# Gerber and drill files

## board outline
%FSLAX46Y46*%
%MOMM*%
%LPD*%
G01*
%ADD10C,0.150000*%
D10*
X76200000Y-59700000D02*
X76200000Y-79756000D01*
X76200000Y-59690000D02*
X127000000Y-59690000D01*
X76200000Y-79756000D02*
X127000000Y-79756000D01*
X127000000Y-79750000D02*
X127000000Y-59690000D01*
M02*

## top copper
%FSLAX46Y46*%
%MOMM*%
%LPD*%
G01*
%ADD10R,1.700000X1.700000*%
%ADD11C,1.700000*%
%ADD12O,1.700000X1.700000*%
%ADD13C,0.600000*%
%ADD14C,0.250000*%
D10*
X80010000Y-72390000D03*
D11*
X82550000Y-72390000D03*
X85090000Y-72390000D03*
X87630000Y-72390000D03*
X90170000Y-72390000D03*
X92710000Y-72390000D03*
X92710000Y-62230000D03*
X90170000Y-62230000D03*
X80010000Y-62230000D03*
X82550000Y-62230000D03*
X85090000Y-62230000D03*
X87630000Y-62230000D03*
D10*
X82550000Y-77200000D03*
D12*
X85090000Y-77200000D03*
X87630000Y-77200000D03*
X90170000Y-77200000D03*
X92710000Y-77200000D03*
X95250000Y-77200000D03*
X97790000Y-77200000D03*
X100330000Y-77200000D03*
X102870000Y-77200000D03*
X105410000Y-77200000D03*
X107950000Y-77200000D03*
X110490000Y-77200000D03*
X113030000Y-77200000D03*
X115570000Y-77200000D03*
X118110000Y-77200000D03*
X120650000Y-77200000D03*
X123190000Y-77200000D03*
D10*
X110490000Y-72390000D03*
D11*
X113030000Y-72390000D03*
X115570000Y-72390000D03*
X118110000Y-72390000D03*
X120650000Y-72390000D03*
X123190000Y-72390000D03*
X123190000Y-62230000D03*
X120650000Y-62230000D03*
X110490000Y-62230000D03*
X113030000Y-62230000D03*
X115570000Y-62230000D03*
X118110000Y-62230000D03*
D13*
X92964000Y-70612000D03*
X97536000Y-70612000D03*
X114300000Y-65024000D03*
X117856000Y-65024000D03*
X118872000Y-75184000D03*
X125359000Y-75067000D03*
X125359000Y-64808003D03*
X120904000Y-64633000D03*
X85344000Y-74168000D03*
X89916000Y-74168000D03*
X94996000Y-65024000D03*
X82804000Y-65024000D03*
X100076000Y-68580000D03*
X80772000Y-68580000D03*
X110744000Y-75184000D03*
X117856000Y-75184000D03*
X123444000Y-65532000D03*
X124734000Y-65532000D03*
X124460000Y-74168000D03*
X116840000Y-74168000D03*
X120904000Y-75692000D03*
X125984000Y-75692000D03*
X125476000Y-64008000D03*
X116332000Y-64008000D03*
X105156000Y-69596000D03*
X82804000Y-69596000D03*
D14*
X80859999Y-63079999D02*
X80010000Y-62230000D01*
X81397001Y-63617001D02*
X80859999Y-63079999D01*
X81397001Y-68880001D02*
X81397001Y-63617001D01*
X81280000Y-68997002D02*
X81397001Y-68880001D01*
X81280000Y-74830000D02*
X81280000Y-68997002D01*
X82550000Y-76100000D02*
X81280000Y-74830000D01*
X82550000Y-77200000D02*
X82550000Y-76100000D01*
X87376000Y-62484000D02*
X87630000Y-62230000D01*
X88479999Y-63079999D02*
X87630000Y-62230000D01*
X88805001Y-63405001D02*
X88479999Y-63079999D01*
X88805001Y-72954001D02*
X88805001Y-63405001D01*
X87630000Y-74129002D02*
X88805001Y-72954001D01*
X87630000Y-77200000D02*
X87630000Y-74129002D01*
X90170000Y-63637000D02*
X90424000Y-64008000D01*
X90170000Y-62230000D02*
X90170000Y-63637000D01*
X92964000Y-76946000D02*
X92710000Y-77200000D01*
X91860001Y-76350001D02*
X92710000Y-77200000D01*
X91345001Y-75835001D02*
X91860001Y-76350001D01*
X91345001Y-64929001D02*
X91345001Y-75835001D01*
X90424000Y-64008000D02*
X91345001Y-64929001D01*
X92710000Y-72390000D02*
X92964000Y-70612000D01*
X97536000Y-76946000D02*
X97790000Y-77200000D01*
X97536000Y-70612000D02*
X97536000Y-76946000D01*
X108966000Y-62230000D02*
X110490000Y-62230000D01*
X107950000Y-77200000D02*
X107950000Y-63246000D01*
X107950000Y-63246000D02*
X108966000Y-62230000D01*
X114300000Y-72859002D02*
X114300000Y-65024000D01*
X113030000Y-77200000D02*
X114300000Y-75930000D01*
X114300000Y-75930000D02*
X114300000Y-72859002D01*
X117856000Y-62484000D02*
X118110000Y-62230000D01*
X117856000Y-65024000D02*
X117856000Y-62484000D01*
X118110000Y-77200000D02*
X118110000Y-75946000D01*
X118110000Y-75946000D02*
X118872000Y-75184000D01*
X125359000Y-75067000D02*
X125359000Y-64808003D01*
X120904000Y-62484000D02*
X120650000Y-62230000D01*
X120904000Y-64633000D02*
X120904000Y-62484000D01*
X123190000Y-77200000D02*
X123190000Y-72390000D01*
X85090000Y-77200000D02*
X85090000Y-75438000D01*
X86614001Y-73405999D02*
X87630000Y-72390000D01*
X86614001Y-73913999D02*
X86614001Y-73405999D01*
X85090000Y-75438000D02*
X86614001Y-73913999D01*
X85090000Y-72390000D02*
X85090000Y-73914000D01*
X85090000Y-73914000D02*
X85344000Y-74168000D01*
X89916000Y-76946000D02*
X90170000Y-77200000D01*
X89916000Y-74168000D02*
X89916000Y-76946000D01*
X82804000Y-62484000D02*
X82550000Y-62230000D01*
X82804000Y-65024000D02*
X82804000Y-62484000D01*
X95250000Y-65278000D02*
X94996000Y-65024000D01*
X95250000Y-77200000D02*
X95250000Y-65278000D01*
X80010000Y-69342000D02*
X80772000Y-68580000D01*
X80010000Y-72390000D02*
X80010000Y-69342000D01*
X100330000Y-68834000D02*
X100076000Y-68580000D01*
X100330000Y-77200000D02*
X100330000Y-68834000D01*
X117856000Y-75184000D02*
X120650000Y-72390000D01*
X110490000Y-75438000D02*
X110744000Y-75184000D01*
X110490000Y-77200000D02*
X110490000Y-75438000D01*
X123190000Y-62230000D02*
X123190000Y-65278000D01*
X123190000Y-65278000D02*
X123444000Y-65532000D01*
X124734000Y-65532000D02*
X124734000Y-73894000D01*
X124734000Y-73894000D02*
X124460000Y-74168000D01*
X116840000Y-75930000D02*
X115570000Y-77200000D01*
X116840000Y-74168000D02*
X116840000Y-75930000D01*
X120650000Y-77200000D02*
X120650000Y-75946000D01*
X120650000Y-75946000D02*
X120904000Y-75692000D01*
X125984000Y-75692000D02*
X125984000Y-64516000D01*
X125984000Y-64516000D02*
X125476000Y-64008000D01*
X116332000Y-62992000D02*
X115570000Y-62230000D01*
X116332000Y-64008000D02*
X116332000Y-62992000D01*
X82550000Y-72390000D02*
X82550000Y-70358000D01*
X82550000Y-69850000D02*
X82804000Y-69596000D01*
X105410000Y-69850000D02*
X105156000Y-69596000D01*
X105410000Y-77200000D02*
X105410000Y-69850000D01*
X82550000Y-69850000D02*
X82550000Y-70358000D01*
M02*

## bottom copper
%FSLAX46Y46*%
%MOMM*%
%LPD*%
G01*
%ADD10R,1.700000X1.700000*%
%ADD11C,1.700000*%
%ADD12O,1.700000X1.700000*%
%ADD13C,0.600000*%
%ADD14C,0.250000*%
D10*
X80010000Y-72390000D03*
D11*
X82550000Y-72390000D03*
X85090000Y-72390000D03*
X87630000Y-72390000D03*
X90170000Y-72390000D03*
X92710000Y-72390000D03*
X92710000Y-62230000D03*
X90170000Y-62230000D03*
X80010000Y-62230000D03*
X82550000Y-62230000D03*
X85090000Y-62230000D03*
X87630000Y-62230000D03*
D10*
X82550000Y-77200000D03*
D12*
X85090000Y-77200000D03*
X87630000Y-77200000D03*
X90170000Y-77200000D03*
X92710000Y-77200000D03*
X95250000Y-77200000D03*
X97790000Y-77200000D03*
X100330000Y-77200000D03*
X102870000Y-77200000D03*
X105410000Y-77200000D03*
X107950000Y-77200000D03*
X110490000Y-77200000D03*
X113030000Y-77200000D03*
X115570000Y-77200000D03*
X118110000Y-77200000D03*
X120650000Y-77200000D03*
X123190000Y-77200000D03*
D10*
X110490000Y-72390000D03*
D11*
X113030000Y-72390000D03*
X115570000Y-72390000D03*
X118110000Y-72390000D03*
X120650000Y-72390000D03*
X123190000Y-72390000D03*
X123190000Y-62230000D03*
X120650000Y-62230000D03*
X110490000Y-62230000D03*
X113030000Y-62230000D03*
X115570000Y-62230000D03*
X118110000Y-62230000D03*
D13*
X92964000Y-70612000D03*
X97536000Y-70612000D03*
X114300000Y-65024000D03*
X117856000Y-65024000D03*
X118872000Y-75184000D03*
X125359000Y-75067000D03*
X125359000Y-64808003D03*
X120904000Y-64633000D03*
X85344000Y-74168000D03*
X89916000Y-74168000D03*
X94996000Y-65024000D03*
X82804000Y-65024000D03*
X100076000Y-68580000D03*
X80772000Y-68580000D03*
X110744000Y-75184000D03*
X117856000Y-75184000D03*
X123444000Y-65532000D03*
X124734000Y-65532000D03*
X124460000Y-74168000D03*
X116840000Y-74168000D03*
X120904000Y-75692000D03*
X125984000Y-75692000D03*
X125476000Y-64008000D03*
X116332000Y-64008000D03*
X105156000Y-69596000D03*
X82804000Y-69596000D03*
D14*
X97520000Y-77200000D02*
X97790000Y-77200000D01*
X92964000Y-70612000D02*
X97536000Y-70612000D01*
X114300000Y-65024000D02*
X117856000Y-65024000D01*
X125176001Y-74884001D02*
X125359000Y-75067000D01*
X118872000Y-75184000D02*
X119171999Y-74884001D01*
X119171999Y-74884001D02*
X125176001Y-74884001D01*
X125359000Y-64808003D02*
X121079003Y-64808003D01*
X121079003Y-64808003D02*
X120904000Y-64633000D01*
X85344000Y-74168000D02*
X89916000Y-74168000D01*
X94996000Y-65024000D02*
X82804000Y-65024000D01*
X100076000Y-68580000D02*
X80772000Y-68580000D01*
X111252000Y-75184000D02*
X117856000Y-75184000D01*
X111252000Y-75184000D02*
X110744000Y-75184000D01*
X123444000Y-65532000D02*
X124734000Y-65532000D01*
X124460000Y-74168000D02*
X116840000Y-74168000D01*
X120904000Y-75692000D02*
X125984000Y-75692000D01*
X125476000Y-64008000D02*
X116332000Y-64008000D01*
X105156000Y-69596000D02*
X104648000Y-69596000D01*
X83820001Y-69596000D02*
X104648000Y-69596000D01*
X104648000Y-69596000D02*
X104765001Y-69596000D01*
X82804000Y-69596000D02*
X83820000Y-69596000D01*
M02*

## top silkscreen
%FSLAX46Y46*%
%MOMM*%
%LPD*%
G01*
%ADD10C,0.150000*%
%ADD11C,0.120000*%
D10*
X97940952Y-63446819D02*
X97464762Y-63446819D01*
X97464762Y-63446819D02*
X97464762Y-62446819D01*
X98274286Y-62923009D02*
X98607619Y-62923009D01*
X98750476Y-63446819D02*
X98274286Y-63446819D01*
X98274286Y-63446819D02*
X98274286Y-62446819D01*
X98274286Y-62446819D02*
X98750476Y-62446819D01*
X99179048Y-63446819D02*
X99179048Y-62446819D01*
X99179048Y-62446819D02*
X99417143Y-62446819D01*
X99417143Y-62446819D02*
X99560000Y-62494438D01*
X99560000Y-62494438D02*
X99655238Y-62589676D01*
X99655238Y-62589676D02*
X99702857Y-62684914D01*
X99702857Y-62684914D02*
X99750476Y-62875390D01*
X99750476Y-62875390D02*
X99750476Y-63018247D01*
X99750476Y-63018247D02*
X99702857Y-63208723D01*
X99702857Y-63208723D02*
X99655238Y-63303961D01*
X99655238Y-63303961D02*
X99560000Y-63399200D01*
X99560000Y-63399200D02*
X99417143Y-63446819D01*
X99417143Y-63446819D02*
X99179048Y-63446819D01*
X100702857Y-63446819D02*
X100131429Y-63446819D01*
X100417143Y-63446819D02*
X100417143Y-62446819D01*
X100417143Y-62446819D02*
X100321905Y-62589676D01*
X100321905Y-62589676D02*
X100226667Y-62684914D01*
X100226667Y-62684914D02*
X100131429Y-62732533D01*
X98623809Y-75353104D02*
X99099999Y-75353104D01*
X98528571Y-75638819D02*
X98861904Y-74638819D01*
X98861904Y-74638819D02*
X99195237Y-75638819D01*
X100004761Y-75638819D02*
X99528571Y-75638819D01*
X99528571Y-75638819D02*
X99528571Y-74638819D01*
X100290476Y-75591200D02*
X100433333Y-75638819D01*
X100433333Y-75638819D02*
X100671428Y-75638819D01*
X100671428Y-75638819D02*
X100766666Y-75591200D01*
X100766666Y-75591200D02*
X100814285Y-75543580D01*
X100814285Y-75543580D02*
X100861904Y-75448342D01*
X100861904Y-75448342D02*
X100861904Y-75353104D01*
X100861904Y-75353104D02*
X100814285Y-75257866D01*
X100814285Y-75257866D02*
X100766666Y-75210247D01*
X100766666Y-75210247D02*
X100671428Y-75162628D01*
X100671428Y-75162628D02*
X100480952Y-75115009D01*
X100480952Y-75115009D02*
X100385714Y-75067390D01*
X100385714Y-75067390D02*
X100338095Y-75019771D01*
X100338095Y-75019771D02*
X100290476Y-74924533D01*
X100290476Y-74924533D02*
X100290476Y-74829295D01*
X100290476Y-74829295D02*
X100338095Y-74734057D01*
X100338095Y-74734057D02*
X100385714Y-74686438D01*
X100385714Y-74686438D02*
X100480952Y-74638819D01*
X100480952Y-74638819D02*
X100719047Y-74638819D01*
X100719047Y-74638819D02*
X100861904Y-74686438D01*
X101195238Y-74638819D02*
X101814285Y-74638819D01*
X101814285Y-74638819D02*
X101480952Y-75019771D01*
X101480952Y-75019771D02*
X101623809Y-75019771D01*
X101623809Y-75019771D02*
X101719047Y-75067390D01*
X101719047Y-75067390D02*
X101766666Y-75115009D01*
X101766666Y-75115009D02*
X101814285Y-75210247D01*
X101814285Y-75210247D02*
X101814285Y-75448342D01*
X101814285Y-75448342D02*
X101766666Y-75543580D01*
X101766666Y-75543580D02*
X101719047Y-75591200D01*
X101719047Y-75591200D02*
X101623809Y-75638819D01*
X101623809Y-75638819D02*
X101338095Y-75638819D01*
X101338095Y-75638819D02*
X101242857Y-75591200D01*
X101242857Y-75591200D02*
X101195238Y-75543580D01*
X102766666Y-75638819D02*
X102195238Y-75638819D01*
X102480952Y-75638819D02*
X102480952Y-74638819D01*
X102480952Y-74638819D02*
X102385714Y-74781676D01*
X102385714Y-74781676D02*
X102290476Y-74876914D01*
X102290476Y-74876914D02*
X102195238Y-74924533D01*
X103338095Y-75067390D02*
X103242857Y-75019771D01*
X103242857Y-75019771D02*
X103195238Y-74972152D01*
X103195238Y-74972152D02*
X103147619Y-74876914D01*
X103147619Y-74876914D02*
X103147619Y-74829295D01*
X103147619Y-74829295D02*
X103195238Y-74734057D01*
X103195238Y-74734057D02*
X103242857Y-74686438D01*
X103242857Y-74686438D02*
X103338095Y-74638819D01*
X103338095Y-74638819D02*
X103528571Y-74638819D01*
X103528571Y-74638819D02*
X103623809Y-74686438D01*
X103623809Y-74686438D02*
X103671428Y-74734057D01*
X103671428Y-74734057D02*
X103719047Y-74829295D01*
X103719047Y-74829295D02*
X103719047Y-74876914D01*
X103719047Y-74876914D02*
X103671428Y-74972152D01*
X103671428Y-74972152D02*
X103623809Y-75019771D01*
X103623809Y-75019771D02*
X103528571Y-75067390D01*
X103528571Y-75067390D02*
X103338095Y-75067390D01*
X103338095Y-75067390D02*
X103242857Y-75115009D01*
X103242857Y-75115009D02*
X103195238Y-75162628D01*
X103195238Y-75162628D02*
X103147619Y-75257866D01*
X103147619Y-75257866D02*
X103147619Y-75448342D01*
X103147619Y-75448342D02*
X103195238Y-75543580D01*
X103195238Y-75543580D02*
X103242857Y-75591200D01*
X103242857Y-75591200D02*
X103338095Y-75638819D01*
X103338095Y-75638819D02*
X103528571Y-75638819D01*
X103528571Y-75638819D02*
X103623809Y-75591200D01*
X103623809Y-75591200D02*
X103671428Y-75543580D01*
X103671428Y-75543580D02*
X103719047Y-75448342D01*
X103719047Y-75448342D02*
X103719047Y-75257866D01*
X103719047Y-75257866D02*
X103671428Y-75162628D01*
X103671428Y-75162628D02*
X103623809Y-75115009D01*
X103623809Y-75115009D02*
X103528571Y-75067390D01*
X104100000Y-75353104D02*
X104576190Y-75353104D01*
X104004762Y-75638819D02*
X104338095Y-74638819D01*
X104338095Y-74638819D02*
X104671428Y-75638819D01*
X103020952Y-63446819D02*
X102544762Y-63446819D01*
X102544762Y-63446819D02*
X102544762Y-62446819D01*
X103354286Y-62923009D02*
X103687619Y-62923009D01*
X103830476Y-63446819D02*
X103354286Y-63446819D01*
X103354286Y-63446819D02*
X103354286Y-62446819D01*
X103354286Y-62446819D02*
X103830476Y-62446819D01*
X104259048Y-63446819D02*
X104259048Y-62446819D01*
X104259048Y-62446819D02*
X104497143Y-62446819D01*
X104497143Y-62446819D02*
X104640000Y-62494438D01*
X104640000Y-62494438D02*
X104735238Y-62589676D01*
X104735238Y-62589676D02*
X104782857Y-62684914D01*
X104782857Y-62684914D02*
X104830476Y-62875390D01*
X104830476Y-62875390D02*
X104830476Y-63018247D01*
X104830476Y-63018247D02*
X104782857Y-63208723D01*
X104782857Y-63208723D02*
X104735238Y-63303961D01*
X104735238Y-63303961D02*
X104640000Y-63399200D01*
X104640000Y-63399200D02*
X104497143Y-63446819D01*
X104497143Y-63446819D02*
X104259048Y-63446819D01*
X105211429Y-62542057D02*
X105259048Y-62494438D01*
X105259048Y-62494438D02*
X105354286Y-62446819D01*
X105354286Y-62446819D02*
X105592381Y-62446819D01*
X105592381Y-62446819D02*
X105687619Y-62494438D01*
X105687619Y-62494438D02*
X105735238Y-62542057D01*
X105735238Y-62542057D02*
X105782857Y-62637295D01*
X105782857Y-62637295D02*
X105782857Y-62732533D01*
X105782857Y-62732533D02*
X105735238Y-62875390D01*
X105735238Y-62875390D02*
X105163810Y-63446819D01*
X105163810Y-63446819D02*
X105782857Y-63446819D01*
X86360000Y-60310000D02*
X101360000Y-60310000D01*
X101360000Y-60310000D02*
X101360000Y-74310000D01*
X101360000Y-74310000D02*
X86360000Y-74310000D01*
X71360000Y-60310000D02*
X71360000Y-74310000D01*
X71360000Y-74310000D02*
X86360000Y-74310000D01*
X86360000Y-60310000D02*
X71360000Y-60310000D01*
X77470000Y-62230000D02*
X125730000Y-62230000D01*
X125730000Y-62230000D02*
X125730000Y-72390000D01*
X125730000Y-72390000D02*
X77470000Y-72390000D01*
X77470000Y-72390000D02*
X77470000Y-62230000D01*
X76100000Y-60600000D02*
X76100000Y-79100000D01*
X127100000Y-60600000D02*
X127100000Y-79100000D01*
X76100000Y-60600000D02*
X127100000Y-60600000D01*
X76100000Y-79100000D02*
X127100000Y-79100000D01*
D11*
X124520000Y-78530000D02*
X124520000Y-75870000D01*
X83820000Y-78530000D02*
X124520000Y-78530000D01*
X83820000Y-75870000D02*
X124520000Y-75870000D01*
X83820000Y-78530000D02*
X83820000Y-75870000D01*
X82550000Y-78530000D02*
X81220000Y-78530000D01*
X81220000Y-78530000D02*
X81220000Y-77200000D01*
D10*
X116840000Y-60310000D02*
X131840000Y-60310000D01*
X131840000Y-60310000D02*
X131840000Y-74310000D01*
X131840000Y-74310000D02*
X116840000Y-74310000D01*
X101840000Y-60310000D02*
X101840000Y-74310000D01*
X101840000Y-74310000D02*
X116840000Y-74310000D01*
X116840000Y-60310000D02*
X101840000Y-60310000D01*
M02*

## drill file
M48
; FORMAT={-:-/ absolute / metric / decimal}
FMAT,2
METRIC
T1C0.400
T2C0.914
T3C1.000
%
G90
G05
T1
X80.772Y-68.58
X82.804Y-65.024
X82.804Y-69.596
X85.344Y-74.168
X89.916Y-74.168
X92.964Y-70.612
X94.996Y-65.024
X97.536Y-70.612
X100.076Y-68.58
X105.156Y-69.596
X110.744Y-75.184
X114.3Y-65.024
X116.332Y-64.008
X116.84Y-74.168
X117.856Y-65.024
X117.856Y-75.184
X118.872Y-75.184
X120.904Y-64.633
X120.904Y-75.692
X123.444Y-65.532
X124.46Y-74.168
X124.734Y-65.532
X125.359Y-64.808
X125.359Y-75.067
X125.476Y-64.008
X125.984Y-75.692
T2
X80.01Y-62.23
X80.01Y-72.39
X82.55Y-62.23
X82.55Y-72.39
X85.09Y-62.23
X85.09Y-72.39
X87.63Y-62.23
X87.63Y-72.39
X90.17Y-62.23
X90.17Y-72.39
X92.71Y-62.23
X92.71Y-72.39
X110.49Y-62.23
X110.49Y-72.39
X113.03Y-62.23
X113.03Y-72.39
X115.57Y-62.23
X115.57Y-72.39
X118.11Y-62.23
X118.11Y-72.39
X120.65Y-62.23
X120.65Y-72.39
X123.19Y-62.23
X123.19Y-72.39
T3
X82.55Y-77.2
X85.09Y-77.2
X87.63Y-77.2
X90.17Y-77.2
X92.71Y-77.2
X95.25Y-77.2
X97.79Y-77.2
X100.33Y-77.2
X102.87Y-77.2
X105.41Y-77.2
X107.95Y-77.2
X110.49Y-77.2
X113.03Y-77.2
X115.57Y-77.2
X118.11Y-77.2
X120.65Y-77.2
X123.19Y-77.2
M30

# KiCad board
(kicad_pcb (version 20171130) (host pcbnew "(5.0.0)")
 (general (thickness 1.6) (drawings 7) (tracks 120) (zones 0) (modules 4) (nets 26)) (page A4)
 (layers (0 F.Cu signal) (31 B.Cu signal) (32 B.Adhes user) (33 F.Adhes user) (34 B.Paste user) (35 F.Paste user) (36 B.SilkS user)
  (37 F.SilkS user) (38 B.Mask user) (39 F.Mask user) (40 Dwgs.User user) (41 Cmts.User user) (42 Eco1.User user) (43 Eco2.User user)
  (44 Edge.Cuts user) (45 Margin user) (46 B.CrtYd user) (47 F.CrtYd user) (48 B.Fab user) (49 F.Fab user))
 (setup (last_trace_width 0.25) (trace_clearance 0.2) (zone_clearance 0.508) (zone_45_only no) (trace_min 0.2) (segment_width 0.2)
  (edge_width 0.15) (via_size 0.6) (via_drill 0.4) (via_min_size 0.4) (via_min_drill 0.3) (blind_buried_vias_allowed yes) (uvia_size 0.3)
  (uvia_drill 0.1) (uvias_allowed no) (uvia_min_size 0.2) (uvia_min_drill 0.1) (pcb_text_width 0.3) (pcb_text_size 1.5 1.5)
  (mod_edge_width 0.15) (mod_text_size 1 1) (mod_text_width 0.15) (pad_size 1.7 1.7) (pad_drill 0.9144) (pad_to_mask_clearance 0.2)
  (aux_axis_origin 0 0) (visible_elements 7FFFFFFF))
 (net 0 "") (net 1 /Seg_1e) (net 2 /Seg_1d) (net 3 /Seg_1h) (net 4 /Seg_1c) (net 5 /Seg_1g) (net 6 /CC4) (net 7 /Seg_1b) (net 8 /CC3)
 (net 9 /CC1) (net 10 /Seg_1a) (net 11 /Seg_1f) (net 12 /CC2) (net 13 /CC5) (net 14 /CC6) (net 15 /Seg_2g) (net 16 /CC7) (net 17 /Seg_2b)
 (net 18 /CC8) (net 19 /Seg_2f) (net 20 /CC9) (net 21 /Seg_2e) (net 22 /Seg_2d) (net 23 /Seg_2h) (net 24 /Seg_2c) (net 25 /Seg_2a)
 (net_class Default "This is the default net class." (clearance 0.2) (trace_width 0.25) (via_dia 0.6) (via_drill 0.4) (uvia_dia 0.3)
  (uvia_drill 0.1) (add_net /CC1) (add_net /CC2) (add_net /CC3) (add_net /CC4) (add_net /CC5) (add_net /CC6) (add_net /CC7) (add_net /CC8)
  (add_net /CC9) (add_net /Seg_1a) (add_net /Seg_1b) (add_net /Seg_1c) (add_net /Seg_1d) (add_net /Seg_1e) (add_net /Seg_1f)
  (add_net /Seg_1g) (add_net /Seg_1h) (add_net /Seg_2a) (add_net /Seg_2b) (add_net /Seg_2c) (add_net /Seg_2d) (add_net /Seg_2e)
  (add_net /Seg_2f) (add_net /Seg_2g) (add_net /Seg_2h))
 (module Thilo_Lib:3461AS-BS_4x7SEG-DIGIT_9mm (layer F.Cu) (at 86.36 67.31)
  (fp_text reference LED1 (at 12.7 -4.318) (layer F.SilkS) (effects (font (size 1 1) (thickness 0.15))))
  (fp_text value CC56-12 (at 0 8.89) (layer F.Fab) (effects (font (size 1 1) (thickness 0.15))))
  (fp_line (start 0 -7) (end 15 -7) (layer F.SilkS) (width 0.15))
  (fp_line (start 15 -7) (end 15 7) (layer F.SilkS) (width 0.15))
  (fp_line (start 15 7) (end 0 7) (layer F.SilkS) (width 0.15))
  (fp_line (start -15 -7) (end -15 7) (layer F.SilkS) (width 0.15))
  (fp_line (start -15 7) (end 0 7) (layer F.SilkS) (width 0.15))
  (fp_line (start 0 -7) (end -15 -7) (layer F.SilkS) (width 0.15))
  (pad 1 thru_hole rect (at -6.35 5.08) (size 1.7 1.7) (drill 0.9144) (layers *.Cu *.Mask) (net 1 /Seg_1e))
  (pad 2 thru_hole circle (at -3.81 5.08) (size 1.7 1.7) (drill 0.9144) (layers *.Cu *.Mask) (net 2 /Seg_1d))
  (pad 3 thru_hole circle (at -1.27 5.08) (size 1.7 1.7) (drill 0.9144) (layers *.Cu *.Mask) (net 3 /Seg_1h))
  (pad 4 thru_hole circle (at 1.27 5.08) (size 1.7 1.7) (drill 0.9144) (layers *.Cu *.Mask) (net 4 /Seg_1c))
  (pad 5 thru_hole circle (at 3.81 5.08) (size 1.7 1.7) (drill 0.9144) (layers *.Cu *.Mask) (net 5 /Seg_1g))
  (pad 6 thru_hole circle (at 6.35 5.08) (size 1.7 1.7) (drill 0.9144) (layers *.Cu *.Mask) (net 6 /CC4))
  (pad 7 thru_hole circle (at 6.35 -5.08) (size 1.7 1.7) (drill 0.9144) (layers *.Cu *.Mask) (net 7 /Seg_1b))
  (pad 8 thru_hole circle (at 3.81 -5.08) (size 1.7 1.7) (drill 0.9144) (layers *.Cu *.Mask) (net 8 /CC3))
  (pad 12 thru_hole circle (at -6.35 -5.08) (size 1.7 1.7) (drill 0.9144) (layers *.Cu *.Mask) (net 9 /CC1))
  (pad 11 thru_hole circle (at -3.81 -5.08) (size 1.7 1.7) (drill 0.9144) (layers *.Cu *.Mask) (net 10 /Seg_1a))
  (pad 10 thru_hole circle (at -1.27 -5.08) (size 1.7 1.7) (drill 0.9144) (layers *.Cu *.Mask) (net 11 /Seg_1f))
  (pad 9 thru_hole circle (at 1.27 -5.08) (size 1.7 1.7) (drill 0.9144) (layers *.Cu *.Mask) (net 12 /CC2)))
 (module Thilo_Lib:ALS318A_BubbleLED (layer F.Cu) (at 101.6 69.85)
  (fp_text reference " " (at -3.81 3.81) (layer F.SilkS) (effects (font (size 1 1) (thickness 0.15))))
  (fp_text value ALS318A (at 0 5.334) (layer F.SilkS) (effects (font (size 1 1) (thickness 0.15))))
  (fp_line (start -24.13 -7.62) (end 24.13 -7.62) (layer F.SilkS) (width 0.15))
  (fp_line (start 24.13 -7.62) (end 24.13 2.54) (layer F.SilkS) (width 0.15))
  (fp_line (start 24.13 2.54) (end -24.13 2.54) (layer F.SilkS) (width 0.15))
  (fp_line (start -24.13 2.54) (end -24.13 -7.62) (layer F.SilkS) (width 0.15))
  (fp_line (start -25.5 -9.25) (end -25.5 9.25) (layer F.SilkS) (width 0.15))
  (fp_line (start 25.5 -9.25) (end 25.5 9.25) (layer F.SilkS) (width 0.15))
  (fp_line (start -25.5 -9.25) (end 25.5 -9.25) (layer F.SilkS) (width 0.15))
  (fp_line (start -25.5 9.25) (end 25.5 9.25) (layer F.SilkS) (width 0.15))
  (fp_line (start 22.92 8.68) (end 22.92 6.02) (layer F.SilkS) (width 0.12))
  (fp_line (start -17.78 8.68) (end 22.92 8.68) (layer F.SilkS) (width 0.12))
  (fp_line (start -17.78 6.02) (end 22.92 6.02) (layer F.SilkS) (width 0.12))
  (fp_line (start -17.78 8.68) (end -17.78 6.02) (layer F.SilkS) (width 0.12))
  (fp_line (start -19.05 8.68) (end -20.38 8.68) (layer F.SilkS) (width 0.12))
  (fp_line (start -20.38 8.68) (end -20.38 7.35) (layer F.SilkS) (width 0.12))
  (pad 1 thru_hole rect (at -19.05 7.35 90) (size 1.7 1.7) (drill 1) (layers *.Cu *.Mask) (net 9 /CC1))
  (pad 2 thru_hole oval (at -16.51 7.35 90) (size 1.7 1.7) (drill 1) (layers *.Cu *.Mask) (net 4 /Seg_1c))
  (pad 3 thru_hole oval (at -13.97 7.35 90) (size 1.7 1.7) (drill 1) (layers *.Cu *.Mask) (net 12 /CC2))
  (pad 4 thru_hole oval (at -11.43 7.35 90) (size 1.7 1.7) (drill 1) (layers *.Cu *.Mask) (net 3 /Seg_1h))
  (pad 5 thru_hole oval (at -8.89 7.35 90) (size 1.7 1.7) (drill 1) (layers *.Cu *.Mask) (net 8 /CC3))
  (pad 6 thru_hole oval (at -6.35 7.35 90) (size 1.7 1.7) (drill 1) (layers *.Cu *.Mask) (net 10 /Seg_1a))
  (pad 7 thru_hole oval (at -3.81 7.35 90) (size 1.7 1.7) (drill 1) (layers *.Cu *.Mask) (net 6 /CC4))
  (pad 8 thru_hole oval (at -1.27 7.35 90) (size 1.7 1.7) (drill 1) (layers *.Cu *.Mask) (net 1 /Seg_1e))
  (pad 9 thru_hole oval (at 1.27 7.35 90) (size 1.7 1.7) (drill 1) (layers *.Cu *.Mask) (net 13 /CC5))
  (pad 10 thru_hole oval (at 3.81 7.35 90) (size 1.7 1.7) (drill 1) (layers *.Cu *.Mask) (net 2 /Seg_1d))
  (pad 11 thru_hole oval (at 6.35 7.35 90) (size 1.7 1.7) (drill 1) (layers *.Cu *.Mask) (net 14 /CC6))
  (pad 12 thru_hole oval (at 8.89 7.35 90) (size 1.7 1.7) (drill 1) (layers *.Cu *.Mask) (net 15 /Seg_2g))
  (pad 13 thru_hole oval (at 11.43 7.35 90) (size 1.7 1.7) (drill 1) (layers *.Cu *.Mask) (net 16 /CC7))
  (pad 14 thru_hole oval (at 13.97 7.35 90) (size 1.7 1.7) (drill 1) (layers *.Cu *.Mask) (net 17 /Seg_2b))
  (pad 15 thru_hole oval (at 16.51 7.35 90) (size 1.7 1.7) (drill 1) (layers *.Cu *.Mask) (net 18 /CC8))
  (pad 16 thru_hole oval (at 19.05 7.35 90) (size 1.7 1.7) (drill 1) (layers *.Cu *.Mask) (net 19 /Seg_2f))
  (pad 17 thru_hole oval (at 21.59 7.35 90) (size 1.7 1.7) (drill 1) (layers *.Cu *.Mask) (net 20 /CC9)))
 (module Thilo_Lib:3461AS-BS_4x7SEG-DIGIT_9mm (layer F.Cu) (at 116.84 67.31)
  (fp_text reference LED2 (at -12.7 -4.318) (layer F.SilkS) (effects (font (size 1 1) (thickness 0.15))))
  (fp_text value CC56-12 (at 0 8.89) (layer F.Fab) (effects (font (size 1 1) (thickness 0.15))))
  (fp_line (start 0 -7) (end 15 -7) (layer F.SilkS) (width 0.15))
  (fp_line (start 15 -7) (end 15 7) (layer F.SilkS) (width 0.15))
  (fp_line (start 15 7) (end 0 7) (layer F.SilkS) (width 0.15))
  (fp_line (start -15 -7) (end -15 7) (layer F.SilkS) (width 0.15))
  (fp_line (start -15 7) (end 0 7) (layer F.SilkS) (width 0.15))
  (fp_line (start 0 -7) (end -15 -7) (layer F.SilkS) (width 0.15))
  (pad 1 thru_hole rect (at -6.35 5.08) (size 1.7 1.7) (drill 0.9144) (layers *.Cu *.Mask) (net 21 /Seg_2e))
  (pad 2 thru_hole circle (at -3.81 5.08) (size 1.7 1.7) (drill 0.9144) (layers *.Cu *.Mask) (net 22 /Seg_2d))
  (pad 3 thru_hole circle (at -1.27 5.08) (size 1.7 1.7) (drill 0.9144) (layers *.Cu *.Mask) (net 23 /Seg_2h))
  (pad 4 thru_hole circle (at 1.27 5.08) (size 1.7 1.7) (drill 0.9144) (layers *.Cu *.Mask) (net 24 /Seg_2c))
  (pad 5 thru_hole circle (at 3.81 5.08) (size 1.7 1.7) (drill 0.9144) (layers *.Cu *.Mask) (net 15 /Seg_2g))
  (pad 6 thru_hole circle (at 6.35 5.08) (size 1.7 1.7) (drill 0.9144) (layers *.Cu *.Mask) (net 20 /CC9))
  (pad 7 thru_hole circle (at 6.35 -5.08) (size 1.7 1.7) (drill 0.9144) (layers *.Cu *.Mask) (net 17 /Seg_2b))
  (pad 8 thru_hole circle (at 3.81 -5.08) (size 1.7 1.7) (drill 0.9144) (layers *.Cu *.Mask) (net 18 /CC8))
  (pad 12 thru_hole circle (at -6.35 -5.08) (size 1.7 1.7) (drill 0.9144) (layers *.Cu *.Mask) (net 14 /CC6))
  (pad 11 thru_hole circle (at -3.81 -5.08) (size 1.7 1.7) (drill 0.9144) (layers *.Cu *.Mask) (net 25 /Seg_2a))
  (pad 10 thru_hole circle (at -1.27 -5.08) (size 1.7 1.7) (drill 0.9144) (layers *.Cu *.Mask) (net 19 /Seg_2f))
  (pad 9 thru_hole circle (at 1.27 -5.08) (size 1.7 1.7) (drill 0.9144) (layers *.Cu *.Mask) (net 16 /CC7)))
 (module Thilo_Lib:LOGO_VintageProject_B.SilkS (layer F.Cu) (at 115.824 69.596)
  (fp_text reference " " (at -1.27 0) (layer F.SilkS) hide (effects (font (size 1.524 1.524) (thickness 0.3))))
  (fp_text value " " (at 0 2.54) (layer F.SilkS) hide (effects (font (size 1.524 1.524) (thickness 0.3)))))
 (gr_line (start 76.2 59.7) (end 76.2 79.756) (layer Edge.Cuts) (width 0.15))
 (gr_line (start 76.2 59.69) (end 127 59.69) (layer Edge.Cuts) (width 0.15))
 (gr_line (start 76.2 79.756) (end 127 79.756) (layer Edge.Cuts) (width 0.15))
 (gr_line (start 127 79.75) (end 127 59.69) (angle 90) (layer Edge.Cuts) (width 0.15))
 (segment (start 80.859999 63.079999) (end 80.01 62.23) (width 0.25) (layer F.Cu) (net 9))
 (segment (start 81.397001 63.617001) (end 80.859999 63.079999) (width 0.25) (layer F.Cu) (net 9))
 (segment (start 81.397001 68.880001) (end 81.397001 63.617001) (width 0.25) (layer F.Cu) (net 9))
 (segment (start 81.28 68.997002) (end 81.397001 68.880001) (width 0.25) (layer F.Cu) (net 9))
 (segment (start 81.28 74.83) (end 81.28 68.997002) (width 0.25) (layer F.Cu) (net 9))
 (segment (start 82.55 76.1) (end 81.28 74.83) (width 0.25) (layer F.Cu) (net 9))
 (segment (start 82.55 77.2) (end 82.55 76.1) (width 0.25) (layer F.Cu) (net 9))
 (segment (start 87.376 62.484) (end 87.63 62.23) (width 0.25) (layer F.Cu) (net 12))
 (segment (start 88.479999 63.079999) (end 87.63 62.23) (width 0.25) (layer F.Cu) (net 12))
 (segment (start 88.805001 63.405001) (end 88.479999 63.079999) (width 0.25) (layer F.Cu) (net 12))
 (segment (start 88.805001 72.954001) (end 88.805001 63.405001) (width 0.25) (layer F.Cu) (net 12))
 (segment (start 87.63 74.129002) (end 88.805001 72.954001) (width 0.25) (layer F.Cu) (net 12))
 (segment (start 87.63 77.2) (end 87.63 74.129002) (width 0.25) (layer F.Cu) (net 12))
 (segment (start 90.17 63.637) (end 90.424 64.008) (width 0.25) (layer F.Cu) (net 8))
 (segment (start 90.17 62.23) (end 90.17 63.637) (width 0.25) (layer F.Cu) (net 8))
 (segment (start 92.964 76.946) (end 92.71 77.2) (width 0.25) (layer F.Cu) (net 8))
 (segment (start 91.860001 76.350001) (end 92.71 77.2) (width 0.25) (layer F.Cu) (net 8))
 (segment (start 91.345001 75.835001) (end 91.860001 76.350001) (width 0.25) (layer F.Cu) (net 8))
 (segment (start 91.345001 64.929001) (end 91.345001 75.835001) (width 0.25) (layer F.Cu) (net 8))
 (segment (start 90.424 64.008) (end 91.345001 64.929001) (width 0.25) (layer F.Cu) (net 8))
 (segment (start 97.52 77.2) (end 97.79 77.2) (width 0.25) (layer B.Cu) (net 6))
 (via blind (at 92.964 70.612) (size 0.6) (drill 0.4) (layers F.Cu B.Cu) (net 6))
 (via blind (at 97.536 70.612) (size 0.6) (drill 0.4) (layers F.Cu B.Cu) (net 6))
 (segment (start 92.964 70.612) (end 97.536 70.612) (width 0.25) (layer B.Cu) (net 6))
 (segment (start 92.71 72.39) (end 92.964 70.612) (width 0.25) (layer F.Cu) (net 6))
 (segment (start 97.536 76.946) (end 97.79 77.2) (width 0.25) (layer F.Cu) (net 6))
 (segment (start 97.536 70.612) (end 97.536 76.946) (width 0.25) (layer F.Cu) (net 6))
 (segment (start 108.966 62.23) (end 110.49 62.23) (width 0.25) (layer F.Cu) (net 14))
 (segment (start 107.95 77.2) (end 107.95 63.246) (width 0.25) (layer F.Cu) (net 14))
 (segment (start 107.95 63.246) (end 108.966 62.23) (width 0.25) (layer F.Cu) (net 14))
 (via blind (at 114.3 65.024) (size 0.6) (drill 0.4) (layers F.Cu B.Cu) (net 16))
 (segment (start 114.3 72.859002) (end 114.3 65.024) (width 0.25) (layer F.Cu) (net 16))
 (segment (start 113.03 77.2) (end 114.3 75.93) (width 0.25) (layer F.Cu) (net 16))
 (segment (start 114.3 75.93) (end 114.3 72.859002) (width 0.25) (layer F.Cu) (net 16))
 (segment (start 114.3 65.024) (end 117.856 65.024) (width 0.25) (layer B.Cu) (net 16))
 (via blind (at 117.856 65.024) (size 0.6) (drill 0.4) (layers F.Cu B.Cu) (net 16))
 (segment (start 117.856 62.484) (end 118.11 62.23) (width 0.25) (layer F.Cu) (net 16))
 (segment (start 117.856 65.024) (end 117.856 62.484) (width 0.25) (layer F.Cu) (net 16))
 (via blind (at 118.872 75.184) (size 0.6) (drill 0.4) (layers F.Cu B.Cu) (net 18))
 (segment (start 118.11 77.2) (end 118.11 75.946) (width 0.25) (layer F.Cu) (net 18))
 (segment (start 118.11 75.946) (end 118.872 75.184) (width 0.25) (layer F.Cu) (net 18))
 (via blind (at 125.359 75.067) (size 0.6) (drill 0.4) (layers F.Cu B.Cu) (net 18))
 (segment (start 125.176001 74.884001) (end 125.359 75.067) (width 0.25) (layer B.Cu) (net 18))
 (segment (start 118.872 75.184) (end 119.171999 74.884001) (width 0.25) (layer B.Cu) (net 18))
 (segment (start 119.171999 74.884001) (end 125.176001 74.884001) (width 0.25) (layer B.Cu) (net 18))
 (via blind (at 125.359 64.808003) (size 0.6) (drill 0.4) (layers F.Cu B.Cu) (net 18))
 (segment (start 125.359 75.067) (end 125.359 64.808003) (width 0.25) (layer F.Cu) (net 18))
 (via blind (at 120.904 64.633) (size 0.6) (drill 0.4) (layers F.Cu B.Cu) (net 18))
 (segment (start 125.359 64.808003) (end 121.079003 64.808003) (width 0.25) (layer B.Cu) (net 18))
 (segment (start 121.079003 64.808003) (end 120.904 64.633) (width 0.25) (layer B.Cu) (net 18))
 (segment (start 120.904 62.484) (end 120.65 62.23) (width 0.25) (layer F.Cu) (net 18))
 (segment (start 120.904 64.633) (end 120.904 62.484) (width 0.25) (layer F.Cu) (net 18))
 (segment (start 123.19 77.2) (end 123.19 72.39) (width 0.25) (layer F.Cu) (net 20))
 (segment (start 85.09 77.2) (end 85.09 75.438) (width 0.25) (layer F.Cu) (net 4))
 (segment (start 86.614001 73.405999) (end 87.63 72.39) (width 0.25) (layer F.Cu) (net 4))
 (segment (start 86.614001 73.913999) (end 86.614001 73.405999) (width 0.25) (layer F.Cu) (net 4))
 (segment (start 85.09 75.438) (end 86.614001 73.913999) (width 0.25) (layer F.Cu) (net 4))
 (via blind (at 85.344 74.168) (size 0.6) (drill 0.4) (layers F.Cu B.Cu) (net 3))
 (segment (start 85.09 72.39) (end 85.09 73.914) (width 0.25) (layer F.Cu) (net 3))
 (segment (start 85.09 73.914) (end 85.344 74.168) (width 0.25) (layer F.Cu) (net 3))
 (via blind (at 89.916 74.168) (size 0.6) (drill 0.4) (layers F.Cu B.Cu) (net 3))
 (segment (start 85.344 74.168) (end 89.916 74.168) (width 0.25) (layer B.Cu) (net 3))
 (segment (start 89.916 76.946) (end 90.17 77.2) (width 0.25) (layer F.Cu) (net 3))
 (segment (start 89.916 74.168) (end 89.916 76.946) (width 0.25) (layer F.Cu) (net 3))
 (via blind (at 94.996 65.024) (size 0.6) (drill 0.4) (layers F.Cu B.Cu) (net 10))
 (via blind (at 82.804 65.024) (size 0.6) (drill 0.4) (layers F.Cu B.Cu) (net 10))
 (segment (start 94.996 65.024) (end 82.804 65.024) (width 0.25) (layer B.Cu) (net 10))
 (segment (start 82.804 62.484) (end 82.55 62.23) (width 0.25) (layer F.Cu) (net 10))
 (segment (start 82.804 65.024) (end 82.804 62.484) (width 0.25) (layer F.Cu) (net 10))
 (segment (start 95.25 65.278) (end 94.996 65.024) (width 0.25) (layer F.Cu) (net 10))
 (segment (start 95.25 77.2) (end 95.25 65.278) (width 0.25) (layer F.Cu) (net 10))
 (via blind (at 100.076 68.58) (size 0.6) (drill 0.4) (layers F.Cu B.Cu) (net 1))
 (via blind (at 80.772 68.58) (size 0.6) (drill 0.4) (layers F.Cu B.Cu) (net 1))
 (segment (start 100.076 68.58) (end 80.772 68.58) (width 0.25) (layer B.Cu) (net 1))
 (segment (start 80.01 69.342) (end 80.772 68.58) (width 0.25) (layer F.Cu) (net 1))
 (segment (start 80.01 72.39) (end 80.01 69.342) (width 0.25) (layer F.Cu) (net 1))
 (segment (start 100.33 68.834) (end 100.076 68.58) (width 0.25) (layer F.Cu) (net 1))
 (segment (start 100.33 77.2) (end 100.33 68.834) (width 0.25) (layer F.Cu) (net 1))
 (via blind (at 110.744 75.184) (size 0.6) (drill 0.4) (layers F.Cu B.Cu) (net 15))
 (via blind (at 117.856 75.184) (size 0.6) (drill 0.4) (layers F.Cu B.Cu) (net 15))
 (segment (start 111.252 75.184) (end 117.856 75.184) (width 0.25) (layer B.Cu) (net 15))
 (segment (start 117.856 75.184) (end 120.65 72.39) (width 0.25) (layer F.Cu) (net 15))
 (segment (start 110.49 75.438) (end 110.744 75.184) (width 0.25) (layer F.Cu) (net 15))
 (segment (start 110.49 77.2) (end 110.49 75.438) (width 0.25) (layer F.Cu) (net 15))
 (segment (start 111.252 75.184) (end 110.744 75.184) (width 0.25) (layer B.Cu) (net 15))
 (via blind (at 123.444 65.532) (size 0.6) (drill 0.4) (layers F.Cu B.Cu) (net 17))
 (segment (start 123.19 62.23) (end 123.19 65.278) (width 0.25) (layer F.Cu) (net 17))
 (segment (start 123.19 65.278) (end 123.444 65.532) (width 0.25) (layer F.Cu) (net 17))
 (via blind (at 124.734 65.532) (size 0.6) (drill 0.4) (layers F.Cu B.Cu) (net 17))
 (segment (start 123.444 65.532) (end 124.734 65.532) (width 0.25) (layer B.Cu) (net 17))
 (via blind (at 124.46 74.168) (size 0.6) (drill 0.4) (layers F.Cu B.Cu) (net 17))
 (segment (start 124.734 65.532) (end 124.734 73.894) (width 0.25) (layer F.Cu) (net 17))
 (segment (start 124.734 73.894) (end 124.46 74.168) (width 0.25) (layer F.Cu) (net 17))
 (via blind (at 116.84 74.168) (size 0.6) (drill 0.4) (layers F.Cu B.Cu) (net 17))
 (segment (start 124.46 74.168) (end 116.84 74.168) (width 0.25) (layer B.Cu) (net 17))
 (segment (start 116.84 75.93) (end 115.57 77.2) (width 0.25) (layer F.Cu) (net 17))
 (segment (start 116.84 74.168) (end 116.84 75.93) (width 0.25) (layer F.Cu) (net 17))
 (via blind (at 120.904 75.692) (size 0.6) (drill 0.4) (layers F.Cu B.Cu) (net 19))
 (segment (start 120.65 77.2) (end 120.65 75.946) (width 0.25) (layer F.Cu) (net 19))
 (segment (start 120.65 75.946) (end 120.904 75.692) (width 0.25) (layer F.Cu) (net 19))
 (via blind (at 125.984 75.692) (size 0.6) (drill 0.4) (layers F.Cu B.Cu) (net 19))
 (segment (start 120.904 75.692) (end 125.984 75.692) (width 0.25) (layer B.Cu) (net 19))
 (via blind (at 125.476 64.008) (size 0.6) (drill 0.4) (layers F.Cu B.Cu) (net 19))
 (segment (start 125.984 75.692) (end 125.984 64.516) (width 0.25) (layer F.Cu) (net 19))
 (segment (start 125.984 64.516) (end 125.476 64.008) (width 0.25) (layer F.Cu) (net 19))
 (via blind (at 116.332 64.008) (size 0.6) (drill 0.4) (layers F.Cu B.Cu) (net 19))
 (segment (start 125.476 64.008) (end 116.332 64.008) (width 0.25) (layer B.Cu) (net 19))
 (segment (start 116.332 62.992) (end 115.57 62.23) (width 0.25) (layer F.Cu) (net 19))
 (segment (start 116.332 64.008) (end 116.332 62.992) (width 0.25) (layer F.Cu) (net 19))
 (via blind (at 105.156 69.596) (size 0.6) (drill 0.4) (layers F.Cu B.Cu) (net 2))
 (segment (start 105.156 69.596) (end 104.648 69.596) (width 0.25) (layer B.Cu) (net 2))
 (segment (start 83.820001 69.596) (end 104.648 69.596) (width 0.25) (layer B.Cu) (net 2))
 (segment (start 104.648 69.596) (end 104.765001 69.596) (width 0.25) (layer B.Cu) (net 2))
 (via blind (at 82.804 69.596) (size 0.6) (drill 0.4) (layers F.Cu B.Cu) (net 2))
 (segment (start 82.55 72.39) (end 82.55 70.358) (width 0.25) (layer F.Cu) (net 2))
 (segment (start 82.55 69.85) (end 82.804 69.596) (width 0.25) (layer F.Cu) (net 2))
 (segment (start 82.804 69.596) (end 83.82 69.596) (width 0.25) (layer B.Cu) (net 2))
 (segment (start 105.41 69.85) (end 105.156 69.596) (width 0.25) (layer F.Cu) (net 2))
 (segment (start 105.41 77.2) (end 105.41 69.85) (width 0.25) (layer F.Cu) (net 2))
 (segment (start 82.55 69.85) (end 82.55 70.358) (width 0.25) (layer F.Cu) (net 2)))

